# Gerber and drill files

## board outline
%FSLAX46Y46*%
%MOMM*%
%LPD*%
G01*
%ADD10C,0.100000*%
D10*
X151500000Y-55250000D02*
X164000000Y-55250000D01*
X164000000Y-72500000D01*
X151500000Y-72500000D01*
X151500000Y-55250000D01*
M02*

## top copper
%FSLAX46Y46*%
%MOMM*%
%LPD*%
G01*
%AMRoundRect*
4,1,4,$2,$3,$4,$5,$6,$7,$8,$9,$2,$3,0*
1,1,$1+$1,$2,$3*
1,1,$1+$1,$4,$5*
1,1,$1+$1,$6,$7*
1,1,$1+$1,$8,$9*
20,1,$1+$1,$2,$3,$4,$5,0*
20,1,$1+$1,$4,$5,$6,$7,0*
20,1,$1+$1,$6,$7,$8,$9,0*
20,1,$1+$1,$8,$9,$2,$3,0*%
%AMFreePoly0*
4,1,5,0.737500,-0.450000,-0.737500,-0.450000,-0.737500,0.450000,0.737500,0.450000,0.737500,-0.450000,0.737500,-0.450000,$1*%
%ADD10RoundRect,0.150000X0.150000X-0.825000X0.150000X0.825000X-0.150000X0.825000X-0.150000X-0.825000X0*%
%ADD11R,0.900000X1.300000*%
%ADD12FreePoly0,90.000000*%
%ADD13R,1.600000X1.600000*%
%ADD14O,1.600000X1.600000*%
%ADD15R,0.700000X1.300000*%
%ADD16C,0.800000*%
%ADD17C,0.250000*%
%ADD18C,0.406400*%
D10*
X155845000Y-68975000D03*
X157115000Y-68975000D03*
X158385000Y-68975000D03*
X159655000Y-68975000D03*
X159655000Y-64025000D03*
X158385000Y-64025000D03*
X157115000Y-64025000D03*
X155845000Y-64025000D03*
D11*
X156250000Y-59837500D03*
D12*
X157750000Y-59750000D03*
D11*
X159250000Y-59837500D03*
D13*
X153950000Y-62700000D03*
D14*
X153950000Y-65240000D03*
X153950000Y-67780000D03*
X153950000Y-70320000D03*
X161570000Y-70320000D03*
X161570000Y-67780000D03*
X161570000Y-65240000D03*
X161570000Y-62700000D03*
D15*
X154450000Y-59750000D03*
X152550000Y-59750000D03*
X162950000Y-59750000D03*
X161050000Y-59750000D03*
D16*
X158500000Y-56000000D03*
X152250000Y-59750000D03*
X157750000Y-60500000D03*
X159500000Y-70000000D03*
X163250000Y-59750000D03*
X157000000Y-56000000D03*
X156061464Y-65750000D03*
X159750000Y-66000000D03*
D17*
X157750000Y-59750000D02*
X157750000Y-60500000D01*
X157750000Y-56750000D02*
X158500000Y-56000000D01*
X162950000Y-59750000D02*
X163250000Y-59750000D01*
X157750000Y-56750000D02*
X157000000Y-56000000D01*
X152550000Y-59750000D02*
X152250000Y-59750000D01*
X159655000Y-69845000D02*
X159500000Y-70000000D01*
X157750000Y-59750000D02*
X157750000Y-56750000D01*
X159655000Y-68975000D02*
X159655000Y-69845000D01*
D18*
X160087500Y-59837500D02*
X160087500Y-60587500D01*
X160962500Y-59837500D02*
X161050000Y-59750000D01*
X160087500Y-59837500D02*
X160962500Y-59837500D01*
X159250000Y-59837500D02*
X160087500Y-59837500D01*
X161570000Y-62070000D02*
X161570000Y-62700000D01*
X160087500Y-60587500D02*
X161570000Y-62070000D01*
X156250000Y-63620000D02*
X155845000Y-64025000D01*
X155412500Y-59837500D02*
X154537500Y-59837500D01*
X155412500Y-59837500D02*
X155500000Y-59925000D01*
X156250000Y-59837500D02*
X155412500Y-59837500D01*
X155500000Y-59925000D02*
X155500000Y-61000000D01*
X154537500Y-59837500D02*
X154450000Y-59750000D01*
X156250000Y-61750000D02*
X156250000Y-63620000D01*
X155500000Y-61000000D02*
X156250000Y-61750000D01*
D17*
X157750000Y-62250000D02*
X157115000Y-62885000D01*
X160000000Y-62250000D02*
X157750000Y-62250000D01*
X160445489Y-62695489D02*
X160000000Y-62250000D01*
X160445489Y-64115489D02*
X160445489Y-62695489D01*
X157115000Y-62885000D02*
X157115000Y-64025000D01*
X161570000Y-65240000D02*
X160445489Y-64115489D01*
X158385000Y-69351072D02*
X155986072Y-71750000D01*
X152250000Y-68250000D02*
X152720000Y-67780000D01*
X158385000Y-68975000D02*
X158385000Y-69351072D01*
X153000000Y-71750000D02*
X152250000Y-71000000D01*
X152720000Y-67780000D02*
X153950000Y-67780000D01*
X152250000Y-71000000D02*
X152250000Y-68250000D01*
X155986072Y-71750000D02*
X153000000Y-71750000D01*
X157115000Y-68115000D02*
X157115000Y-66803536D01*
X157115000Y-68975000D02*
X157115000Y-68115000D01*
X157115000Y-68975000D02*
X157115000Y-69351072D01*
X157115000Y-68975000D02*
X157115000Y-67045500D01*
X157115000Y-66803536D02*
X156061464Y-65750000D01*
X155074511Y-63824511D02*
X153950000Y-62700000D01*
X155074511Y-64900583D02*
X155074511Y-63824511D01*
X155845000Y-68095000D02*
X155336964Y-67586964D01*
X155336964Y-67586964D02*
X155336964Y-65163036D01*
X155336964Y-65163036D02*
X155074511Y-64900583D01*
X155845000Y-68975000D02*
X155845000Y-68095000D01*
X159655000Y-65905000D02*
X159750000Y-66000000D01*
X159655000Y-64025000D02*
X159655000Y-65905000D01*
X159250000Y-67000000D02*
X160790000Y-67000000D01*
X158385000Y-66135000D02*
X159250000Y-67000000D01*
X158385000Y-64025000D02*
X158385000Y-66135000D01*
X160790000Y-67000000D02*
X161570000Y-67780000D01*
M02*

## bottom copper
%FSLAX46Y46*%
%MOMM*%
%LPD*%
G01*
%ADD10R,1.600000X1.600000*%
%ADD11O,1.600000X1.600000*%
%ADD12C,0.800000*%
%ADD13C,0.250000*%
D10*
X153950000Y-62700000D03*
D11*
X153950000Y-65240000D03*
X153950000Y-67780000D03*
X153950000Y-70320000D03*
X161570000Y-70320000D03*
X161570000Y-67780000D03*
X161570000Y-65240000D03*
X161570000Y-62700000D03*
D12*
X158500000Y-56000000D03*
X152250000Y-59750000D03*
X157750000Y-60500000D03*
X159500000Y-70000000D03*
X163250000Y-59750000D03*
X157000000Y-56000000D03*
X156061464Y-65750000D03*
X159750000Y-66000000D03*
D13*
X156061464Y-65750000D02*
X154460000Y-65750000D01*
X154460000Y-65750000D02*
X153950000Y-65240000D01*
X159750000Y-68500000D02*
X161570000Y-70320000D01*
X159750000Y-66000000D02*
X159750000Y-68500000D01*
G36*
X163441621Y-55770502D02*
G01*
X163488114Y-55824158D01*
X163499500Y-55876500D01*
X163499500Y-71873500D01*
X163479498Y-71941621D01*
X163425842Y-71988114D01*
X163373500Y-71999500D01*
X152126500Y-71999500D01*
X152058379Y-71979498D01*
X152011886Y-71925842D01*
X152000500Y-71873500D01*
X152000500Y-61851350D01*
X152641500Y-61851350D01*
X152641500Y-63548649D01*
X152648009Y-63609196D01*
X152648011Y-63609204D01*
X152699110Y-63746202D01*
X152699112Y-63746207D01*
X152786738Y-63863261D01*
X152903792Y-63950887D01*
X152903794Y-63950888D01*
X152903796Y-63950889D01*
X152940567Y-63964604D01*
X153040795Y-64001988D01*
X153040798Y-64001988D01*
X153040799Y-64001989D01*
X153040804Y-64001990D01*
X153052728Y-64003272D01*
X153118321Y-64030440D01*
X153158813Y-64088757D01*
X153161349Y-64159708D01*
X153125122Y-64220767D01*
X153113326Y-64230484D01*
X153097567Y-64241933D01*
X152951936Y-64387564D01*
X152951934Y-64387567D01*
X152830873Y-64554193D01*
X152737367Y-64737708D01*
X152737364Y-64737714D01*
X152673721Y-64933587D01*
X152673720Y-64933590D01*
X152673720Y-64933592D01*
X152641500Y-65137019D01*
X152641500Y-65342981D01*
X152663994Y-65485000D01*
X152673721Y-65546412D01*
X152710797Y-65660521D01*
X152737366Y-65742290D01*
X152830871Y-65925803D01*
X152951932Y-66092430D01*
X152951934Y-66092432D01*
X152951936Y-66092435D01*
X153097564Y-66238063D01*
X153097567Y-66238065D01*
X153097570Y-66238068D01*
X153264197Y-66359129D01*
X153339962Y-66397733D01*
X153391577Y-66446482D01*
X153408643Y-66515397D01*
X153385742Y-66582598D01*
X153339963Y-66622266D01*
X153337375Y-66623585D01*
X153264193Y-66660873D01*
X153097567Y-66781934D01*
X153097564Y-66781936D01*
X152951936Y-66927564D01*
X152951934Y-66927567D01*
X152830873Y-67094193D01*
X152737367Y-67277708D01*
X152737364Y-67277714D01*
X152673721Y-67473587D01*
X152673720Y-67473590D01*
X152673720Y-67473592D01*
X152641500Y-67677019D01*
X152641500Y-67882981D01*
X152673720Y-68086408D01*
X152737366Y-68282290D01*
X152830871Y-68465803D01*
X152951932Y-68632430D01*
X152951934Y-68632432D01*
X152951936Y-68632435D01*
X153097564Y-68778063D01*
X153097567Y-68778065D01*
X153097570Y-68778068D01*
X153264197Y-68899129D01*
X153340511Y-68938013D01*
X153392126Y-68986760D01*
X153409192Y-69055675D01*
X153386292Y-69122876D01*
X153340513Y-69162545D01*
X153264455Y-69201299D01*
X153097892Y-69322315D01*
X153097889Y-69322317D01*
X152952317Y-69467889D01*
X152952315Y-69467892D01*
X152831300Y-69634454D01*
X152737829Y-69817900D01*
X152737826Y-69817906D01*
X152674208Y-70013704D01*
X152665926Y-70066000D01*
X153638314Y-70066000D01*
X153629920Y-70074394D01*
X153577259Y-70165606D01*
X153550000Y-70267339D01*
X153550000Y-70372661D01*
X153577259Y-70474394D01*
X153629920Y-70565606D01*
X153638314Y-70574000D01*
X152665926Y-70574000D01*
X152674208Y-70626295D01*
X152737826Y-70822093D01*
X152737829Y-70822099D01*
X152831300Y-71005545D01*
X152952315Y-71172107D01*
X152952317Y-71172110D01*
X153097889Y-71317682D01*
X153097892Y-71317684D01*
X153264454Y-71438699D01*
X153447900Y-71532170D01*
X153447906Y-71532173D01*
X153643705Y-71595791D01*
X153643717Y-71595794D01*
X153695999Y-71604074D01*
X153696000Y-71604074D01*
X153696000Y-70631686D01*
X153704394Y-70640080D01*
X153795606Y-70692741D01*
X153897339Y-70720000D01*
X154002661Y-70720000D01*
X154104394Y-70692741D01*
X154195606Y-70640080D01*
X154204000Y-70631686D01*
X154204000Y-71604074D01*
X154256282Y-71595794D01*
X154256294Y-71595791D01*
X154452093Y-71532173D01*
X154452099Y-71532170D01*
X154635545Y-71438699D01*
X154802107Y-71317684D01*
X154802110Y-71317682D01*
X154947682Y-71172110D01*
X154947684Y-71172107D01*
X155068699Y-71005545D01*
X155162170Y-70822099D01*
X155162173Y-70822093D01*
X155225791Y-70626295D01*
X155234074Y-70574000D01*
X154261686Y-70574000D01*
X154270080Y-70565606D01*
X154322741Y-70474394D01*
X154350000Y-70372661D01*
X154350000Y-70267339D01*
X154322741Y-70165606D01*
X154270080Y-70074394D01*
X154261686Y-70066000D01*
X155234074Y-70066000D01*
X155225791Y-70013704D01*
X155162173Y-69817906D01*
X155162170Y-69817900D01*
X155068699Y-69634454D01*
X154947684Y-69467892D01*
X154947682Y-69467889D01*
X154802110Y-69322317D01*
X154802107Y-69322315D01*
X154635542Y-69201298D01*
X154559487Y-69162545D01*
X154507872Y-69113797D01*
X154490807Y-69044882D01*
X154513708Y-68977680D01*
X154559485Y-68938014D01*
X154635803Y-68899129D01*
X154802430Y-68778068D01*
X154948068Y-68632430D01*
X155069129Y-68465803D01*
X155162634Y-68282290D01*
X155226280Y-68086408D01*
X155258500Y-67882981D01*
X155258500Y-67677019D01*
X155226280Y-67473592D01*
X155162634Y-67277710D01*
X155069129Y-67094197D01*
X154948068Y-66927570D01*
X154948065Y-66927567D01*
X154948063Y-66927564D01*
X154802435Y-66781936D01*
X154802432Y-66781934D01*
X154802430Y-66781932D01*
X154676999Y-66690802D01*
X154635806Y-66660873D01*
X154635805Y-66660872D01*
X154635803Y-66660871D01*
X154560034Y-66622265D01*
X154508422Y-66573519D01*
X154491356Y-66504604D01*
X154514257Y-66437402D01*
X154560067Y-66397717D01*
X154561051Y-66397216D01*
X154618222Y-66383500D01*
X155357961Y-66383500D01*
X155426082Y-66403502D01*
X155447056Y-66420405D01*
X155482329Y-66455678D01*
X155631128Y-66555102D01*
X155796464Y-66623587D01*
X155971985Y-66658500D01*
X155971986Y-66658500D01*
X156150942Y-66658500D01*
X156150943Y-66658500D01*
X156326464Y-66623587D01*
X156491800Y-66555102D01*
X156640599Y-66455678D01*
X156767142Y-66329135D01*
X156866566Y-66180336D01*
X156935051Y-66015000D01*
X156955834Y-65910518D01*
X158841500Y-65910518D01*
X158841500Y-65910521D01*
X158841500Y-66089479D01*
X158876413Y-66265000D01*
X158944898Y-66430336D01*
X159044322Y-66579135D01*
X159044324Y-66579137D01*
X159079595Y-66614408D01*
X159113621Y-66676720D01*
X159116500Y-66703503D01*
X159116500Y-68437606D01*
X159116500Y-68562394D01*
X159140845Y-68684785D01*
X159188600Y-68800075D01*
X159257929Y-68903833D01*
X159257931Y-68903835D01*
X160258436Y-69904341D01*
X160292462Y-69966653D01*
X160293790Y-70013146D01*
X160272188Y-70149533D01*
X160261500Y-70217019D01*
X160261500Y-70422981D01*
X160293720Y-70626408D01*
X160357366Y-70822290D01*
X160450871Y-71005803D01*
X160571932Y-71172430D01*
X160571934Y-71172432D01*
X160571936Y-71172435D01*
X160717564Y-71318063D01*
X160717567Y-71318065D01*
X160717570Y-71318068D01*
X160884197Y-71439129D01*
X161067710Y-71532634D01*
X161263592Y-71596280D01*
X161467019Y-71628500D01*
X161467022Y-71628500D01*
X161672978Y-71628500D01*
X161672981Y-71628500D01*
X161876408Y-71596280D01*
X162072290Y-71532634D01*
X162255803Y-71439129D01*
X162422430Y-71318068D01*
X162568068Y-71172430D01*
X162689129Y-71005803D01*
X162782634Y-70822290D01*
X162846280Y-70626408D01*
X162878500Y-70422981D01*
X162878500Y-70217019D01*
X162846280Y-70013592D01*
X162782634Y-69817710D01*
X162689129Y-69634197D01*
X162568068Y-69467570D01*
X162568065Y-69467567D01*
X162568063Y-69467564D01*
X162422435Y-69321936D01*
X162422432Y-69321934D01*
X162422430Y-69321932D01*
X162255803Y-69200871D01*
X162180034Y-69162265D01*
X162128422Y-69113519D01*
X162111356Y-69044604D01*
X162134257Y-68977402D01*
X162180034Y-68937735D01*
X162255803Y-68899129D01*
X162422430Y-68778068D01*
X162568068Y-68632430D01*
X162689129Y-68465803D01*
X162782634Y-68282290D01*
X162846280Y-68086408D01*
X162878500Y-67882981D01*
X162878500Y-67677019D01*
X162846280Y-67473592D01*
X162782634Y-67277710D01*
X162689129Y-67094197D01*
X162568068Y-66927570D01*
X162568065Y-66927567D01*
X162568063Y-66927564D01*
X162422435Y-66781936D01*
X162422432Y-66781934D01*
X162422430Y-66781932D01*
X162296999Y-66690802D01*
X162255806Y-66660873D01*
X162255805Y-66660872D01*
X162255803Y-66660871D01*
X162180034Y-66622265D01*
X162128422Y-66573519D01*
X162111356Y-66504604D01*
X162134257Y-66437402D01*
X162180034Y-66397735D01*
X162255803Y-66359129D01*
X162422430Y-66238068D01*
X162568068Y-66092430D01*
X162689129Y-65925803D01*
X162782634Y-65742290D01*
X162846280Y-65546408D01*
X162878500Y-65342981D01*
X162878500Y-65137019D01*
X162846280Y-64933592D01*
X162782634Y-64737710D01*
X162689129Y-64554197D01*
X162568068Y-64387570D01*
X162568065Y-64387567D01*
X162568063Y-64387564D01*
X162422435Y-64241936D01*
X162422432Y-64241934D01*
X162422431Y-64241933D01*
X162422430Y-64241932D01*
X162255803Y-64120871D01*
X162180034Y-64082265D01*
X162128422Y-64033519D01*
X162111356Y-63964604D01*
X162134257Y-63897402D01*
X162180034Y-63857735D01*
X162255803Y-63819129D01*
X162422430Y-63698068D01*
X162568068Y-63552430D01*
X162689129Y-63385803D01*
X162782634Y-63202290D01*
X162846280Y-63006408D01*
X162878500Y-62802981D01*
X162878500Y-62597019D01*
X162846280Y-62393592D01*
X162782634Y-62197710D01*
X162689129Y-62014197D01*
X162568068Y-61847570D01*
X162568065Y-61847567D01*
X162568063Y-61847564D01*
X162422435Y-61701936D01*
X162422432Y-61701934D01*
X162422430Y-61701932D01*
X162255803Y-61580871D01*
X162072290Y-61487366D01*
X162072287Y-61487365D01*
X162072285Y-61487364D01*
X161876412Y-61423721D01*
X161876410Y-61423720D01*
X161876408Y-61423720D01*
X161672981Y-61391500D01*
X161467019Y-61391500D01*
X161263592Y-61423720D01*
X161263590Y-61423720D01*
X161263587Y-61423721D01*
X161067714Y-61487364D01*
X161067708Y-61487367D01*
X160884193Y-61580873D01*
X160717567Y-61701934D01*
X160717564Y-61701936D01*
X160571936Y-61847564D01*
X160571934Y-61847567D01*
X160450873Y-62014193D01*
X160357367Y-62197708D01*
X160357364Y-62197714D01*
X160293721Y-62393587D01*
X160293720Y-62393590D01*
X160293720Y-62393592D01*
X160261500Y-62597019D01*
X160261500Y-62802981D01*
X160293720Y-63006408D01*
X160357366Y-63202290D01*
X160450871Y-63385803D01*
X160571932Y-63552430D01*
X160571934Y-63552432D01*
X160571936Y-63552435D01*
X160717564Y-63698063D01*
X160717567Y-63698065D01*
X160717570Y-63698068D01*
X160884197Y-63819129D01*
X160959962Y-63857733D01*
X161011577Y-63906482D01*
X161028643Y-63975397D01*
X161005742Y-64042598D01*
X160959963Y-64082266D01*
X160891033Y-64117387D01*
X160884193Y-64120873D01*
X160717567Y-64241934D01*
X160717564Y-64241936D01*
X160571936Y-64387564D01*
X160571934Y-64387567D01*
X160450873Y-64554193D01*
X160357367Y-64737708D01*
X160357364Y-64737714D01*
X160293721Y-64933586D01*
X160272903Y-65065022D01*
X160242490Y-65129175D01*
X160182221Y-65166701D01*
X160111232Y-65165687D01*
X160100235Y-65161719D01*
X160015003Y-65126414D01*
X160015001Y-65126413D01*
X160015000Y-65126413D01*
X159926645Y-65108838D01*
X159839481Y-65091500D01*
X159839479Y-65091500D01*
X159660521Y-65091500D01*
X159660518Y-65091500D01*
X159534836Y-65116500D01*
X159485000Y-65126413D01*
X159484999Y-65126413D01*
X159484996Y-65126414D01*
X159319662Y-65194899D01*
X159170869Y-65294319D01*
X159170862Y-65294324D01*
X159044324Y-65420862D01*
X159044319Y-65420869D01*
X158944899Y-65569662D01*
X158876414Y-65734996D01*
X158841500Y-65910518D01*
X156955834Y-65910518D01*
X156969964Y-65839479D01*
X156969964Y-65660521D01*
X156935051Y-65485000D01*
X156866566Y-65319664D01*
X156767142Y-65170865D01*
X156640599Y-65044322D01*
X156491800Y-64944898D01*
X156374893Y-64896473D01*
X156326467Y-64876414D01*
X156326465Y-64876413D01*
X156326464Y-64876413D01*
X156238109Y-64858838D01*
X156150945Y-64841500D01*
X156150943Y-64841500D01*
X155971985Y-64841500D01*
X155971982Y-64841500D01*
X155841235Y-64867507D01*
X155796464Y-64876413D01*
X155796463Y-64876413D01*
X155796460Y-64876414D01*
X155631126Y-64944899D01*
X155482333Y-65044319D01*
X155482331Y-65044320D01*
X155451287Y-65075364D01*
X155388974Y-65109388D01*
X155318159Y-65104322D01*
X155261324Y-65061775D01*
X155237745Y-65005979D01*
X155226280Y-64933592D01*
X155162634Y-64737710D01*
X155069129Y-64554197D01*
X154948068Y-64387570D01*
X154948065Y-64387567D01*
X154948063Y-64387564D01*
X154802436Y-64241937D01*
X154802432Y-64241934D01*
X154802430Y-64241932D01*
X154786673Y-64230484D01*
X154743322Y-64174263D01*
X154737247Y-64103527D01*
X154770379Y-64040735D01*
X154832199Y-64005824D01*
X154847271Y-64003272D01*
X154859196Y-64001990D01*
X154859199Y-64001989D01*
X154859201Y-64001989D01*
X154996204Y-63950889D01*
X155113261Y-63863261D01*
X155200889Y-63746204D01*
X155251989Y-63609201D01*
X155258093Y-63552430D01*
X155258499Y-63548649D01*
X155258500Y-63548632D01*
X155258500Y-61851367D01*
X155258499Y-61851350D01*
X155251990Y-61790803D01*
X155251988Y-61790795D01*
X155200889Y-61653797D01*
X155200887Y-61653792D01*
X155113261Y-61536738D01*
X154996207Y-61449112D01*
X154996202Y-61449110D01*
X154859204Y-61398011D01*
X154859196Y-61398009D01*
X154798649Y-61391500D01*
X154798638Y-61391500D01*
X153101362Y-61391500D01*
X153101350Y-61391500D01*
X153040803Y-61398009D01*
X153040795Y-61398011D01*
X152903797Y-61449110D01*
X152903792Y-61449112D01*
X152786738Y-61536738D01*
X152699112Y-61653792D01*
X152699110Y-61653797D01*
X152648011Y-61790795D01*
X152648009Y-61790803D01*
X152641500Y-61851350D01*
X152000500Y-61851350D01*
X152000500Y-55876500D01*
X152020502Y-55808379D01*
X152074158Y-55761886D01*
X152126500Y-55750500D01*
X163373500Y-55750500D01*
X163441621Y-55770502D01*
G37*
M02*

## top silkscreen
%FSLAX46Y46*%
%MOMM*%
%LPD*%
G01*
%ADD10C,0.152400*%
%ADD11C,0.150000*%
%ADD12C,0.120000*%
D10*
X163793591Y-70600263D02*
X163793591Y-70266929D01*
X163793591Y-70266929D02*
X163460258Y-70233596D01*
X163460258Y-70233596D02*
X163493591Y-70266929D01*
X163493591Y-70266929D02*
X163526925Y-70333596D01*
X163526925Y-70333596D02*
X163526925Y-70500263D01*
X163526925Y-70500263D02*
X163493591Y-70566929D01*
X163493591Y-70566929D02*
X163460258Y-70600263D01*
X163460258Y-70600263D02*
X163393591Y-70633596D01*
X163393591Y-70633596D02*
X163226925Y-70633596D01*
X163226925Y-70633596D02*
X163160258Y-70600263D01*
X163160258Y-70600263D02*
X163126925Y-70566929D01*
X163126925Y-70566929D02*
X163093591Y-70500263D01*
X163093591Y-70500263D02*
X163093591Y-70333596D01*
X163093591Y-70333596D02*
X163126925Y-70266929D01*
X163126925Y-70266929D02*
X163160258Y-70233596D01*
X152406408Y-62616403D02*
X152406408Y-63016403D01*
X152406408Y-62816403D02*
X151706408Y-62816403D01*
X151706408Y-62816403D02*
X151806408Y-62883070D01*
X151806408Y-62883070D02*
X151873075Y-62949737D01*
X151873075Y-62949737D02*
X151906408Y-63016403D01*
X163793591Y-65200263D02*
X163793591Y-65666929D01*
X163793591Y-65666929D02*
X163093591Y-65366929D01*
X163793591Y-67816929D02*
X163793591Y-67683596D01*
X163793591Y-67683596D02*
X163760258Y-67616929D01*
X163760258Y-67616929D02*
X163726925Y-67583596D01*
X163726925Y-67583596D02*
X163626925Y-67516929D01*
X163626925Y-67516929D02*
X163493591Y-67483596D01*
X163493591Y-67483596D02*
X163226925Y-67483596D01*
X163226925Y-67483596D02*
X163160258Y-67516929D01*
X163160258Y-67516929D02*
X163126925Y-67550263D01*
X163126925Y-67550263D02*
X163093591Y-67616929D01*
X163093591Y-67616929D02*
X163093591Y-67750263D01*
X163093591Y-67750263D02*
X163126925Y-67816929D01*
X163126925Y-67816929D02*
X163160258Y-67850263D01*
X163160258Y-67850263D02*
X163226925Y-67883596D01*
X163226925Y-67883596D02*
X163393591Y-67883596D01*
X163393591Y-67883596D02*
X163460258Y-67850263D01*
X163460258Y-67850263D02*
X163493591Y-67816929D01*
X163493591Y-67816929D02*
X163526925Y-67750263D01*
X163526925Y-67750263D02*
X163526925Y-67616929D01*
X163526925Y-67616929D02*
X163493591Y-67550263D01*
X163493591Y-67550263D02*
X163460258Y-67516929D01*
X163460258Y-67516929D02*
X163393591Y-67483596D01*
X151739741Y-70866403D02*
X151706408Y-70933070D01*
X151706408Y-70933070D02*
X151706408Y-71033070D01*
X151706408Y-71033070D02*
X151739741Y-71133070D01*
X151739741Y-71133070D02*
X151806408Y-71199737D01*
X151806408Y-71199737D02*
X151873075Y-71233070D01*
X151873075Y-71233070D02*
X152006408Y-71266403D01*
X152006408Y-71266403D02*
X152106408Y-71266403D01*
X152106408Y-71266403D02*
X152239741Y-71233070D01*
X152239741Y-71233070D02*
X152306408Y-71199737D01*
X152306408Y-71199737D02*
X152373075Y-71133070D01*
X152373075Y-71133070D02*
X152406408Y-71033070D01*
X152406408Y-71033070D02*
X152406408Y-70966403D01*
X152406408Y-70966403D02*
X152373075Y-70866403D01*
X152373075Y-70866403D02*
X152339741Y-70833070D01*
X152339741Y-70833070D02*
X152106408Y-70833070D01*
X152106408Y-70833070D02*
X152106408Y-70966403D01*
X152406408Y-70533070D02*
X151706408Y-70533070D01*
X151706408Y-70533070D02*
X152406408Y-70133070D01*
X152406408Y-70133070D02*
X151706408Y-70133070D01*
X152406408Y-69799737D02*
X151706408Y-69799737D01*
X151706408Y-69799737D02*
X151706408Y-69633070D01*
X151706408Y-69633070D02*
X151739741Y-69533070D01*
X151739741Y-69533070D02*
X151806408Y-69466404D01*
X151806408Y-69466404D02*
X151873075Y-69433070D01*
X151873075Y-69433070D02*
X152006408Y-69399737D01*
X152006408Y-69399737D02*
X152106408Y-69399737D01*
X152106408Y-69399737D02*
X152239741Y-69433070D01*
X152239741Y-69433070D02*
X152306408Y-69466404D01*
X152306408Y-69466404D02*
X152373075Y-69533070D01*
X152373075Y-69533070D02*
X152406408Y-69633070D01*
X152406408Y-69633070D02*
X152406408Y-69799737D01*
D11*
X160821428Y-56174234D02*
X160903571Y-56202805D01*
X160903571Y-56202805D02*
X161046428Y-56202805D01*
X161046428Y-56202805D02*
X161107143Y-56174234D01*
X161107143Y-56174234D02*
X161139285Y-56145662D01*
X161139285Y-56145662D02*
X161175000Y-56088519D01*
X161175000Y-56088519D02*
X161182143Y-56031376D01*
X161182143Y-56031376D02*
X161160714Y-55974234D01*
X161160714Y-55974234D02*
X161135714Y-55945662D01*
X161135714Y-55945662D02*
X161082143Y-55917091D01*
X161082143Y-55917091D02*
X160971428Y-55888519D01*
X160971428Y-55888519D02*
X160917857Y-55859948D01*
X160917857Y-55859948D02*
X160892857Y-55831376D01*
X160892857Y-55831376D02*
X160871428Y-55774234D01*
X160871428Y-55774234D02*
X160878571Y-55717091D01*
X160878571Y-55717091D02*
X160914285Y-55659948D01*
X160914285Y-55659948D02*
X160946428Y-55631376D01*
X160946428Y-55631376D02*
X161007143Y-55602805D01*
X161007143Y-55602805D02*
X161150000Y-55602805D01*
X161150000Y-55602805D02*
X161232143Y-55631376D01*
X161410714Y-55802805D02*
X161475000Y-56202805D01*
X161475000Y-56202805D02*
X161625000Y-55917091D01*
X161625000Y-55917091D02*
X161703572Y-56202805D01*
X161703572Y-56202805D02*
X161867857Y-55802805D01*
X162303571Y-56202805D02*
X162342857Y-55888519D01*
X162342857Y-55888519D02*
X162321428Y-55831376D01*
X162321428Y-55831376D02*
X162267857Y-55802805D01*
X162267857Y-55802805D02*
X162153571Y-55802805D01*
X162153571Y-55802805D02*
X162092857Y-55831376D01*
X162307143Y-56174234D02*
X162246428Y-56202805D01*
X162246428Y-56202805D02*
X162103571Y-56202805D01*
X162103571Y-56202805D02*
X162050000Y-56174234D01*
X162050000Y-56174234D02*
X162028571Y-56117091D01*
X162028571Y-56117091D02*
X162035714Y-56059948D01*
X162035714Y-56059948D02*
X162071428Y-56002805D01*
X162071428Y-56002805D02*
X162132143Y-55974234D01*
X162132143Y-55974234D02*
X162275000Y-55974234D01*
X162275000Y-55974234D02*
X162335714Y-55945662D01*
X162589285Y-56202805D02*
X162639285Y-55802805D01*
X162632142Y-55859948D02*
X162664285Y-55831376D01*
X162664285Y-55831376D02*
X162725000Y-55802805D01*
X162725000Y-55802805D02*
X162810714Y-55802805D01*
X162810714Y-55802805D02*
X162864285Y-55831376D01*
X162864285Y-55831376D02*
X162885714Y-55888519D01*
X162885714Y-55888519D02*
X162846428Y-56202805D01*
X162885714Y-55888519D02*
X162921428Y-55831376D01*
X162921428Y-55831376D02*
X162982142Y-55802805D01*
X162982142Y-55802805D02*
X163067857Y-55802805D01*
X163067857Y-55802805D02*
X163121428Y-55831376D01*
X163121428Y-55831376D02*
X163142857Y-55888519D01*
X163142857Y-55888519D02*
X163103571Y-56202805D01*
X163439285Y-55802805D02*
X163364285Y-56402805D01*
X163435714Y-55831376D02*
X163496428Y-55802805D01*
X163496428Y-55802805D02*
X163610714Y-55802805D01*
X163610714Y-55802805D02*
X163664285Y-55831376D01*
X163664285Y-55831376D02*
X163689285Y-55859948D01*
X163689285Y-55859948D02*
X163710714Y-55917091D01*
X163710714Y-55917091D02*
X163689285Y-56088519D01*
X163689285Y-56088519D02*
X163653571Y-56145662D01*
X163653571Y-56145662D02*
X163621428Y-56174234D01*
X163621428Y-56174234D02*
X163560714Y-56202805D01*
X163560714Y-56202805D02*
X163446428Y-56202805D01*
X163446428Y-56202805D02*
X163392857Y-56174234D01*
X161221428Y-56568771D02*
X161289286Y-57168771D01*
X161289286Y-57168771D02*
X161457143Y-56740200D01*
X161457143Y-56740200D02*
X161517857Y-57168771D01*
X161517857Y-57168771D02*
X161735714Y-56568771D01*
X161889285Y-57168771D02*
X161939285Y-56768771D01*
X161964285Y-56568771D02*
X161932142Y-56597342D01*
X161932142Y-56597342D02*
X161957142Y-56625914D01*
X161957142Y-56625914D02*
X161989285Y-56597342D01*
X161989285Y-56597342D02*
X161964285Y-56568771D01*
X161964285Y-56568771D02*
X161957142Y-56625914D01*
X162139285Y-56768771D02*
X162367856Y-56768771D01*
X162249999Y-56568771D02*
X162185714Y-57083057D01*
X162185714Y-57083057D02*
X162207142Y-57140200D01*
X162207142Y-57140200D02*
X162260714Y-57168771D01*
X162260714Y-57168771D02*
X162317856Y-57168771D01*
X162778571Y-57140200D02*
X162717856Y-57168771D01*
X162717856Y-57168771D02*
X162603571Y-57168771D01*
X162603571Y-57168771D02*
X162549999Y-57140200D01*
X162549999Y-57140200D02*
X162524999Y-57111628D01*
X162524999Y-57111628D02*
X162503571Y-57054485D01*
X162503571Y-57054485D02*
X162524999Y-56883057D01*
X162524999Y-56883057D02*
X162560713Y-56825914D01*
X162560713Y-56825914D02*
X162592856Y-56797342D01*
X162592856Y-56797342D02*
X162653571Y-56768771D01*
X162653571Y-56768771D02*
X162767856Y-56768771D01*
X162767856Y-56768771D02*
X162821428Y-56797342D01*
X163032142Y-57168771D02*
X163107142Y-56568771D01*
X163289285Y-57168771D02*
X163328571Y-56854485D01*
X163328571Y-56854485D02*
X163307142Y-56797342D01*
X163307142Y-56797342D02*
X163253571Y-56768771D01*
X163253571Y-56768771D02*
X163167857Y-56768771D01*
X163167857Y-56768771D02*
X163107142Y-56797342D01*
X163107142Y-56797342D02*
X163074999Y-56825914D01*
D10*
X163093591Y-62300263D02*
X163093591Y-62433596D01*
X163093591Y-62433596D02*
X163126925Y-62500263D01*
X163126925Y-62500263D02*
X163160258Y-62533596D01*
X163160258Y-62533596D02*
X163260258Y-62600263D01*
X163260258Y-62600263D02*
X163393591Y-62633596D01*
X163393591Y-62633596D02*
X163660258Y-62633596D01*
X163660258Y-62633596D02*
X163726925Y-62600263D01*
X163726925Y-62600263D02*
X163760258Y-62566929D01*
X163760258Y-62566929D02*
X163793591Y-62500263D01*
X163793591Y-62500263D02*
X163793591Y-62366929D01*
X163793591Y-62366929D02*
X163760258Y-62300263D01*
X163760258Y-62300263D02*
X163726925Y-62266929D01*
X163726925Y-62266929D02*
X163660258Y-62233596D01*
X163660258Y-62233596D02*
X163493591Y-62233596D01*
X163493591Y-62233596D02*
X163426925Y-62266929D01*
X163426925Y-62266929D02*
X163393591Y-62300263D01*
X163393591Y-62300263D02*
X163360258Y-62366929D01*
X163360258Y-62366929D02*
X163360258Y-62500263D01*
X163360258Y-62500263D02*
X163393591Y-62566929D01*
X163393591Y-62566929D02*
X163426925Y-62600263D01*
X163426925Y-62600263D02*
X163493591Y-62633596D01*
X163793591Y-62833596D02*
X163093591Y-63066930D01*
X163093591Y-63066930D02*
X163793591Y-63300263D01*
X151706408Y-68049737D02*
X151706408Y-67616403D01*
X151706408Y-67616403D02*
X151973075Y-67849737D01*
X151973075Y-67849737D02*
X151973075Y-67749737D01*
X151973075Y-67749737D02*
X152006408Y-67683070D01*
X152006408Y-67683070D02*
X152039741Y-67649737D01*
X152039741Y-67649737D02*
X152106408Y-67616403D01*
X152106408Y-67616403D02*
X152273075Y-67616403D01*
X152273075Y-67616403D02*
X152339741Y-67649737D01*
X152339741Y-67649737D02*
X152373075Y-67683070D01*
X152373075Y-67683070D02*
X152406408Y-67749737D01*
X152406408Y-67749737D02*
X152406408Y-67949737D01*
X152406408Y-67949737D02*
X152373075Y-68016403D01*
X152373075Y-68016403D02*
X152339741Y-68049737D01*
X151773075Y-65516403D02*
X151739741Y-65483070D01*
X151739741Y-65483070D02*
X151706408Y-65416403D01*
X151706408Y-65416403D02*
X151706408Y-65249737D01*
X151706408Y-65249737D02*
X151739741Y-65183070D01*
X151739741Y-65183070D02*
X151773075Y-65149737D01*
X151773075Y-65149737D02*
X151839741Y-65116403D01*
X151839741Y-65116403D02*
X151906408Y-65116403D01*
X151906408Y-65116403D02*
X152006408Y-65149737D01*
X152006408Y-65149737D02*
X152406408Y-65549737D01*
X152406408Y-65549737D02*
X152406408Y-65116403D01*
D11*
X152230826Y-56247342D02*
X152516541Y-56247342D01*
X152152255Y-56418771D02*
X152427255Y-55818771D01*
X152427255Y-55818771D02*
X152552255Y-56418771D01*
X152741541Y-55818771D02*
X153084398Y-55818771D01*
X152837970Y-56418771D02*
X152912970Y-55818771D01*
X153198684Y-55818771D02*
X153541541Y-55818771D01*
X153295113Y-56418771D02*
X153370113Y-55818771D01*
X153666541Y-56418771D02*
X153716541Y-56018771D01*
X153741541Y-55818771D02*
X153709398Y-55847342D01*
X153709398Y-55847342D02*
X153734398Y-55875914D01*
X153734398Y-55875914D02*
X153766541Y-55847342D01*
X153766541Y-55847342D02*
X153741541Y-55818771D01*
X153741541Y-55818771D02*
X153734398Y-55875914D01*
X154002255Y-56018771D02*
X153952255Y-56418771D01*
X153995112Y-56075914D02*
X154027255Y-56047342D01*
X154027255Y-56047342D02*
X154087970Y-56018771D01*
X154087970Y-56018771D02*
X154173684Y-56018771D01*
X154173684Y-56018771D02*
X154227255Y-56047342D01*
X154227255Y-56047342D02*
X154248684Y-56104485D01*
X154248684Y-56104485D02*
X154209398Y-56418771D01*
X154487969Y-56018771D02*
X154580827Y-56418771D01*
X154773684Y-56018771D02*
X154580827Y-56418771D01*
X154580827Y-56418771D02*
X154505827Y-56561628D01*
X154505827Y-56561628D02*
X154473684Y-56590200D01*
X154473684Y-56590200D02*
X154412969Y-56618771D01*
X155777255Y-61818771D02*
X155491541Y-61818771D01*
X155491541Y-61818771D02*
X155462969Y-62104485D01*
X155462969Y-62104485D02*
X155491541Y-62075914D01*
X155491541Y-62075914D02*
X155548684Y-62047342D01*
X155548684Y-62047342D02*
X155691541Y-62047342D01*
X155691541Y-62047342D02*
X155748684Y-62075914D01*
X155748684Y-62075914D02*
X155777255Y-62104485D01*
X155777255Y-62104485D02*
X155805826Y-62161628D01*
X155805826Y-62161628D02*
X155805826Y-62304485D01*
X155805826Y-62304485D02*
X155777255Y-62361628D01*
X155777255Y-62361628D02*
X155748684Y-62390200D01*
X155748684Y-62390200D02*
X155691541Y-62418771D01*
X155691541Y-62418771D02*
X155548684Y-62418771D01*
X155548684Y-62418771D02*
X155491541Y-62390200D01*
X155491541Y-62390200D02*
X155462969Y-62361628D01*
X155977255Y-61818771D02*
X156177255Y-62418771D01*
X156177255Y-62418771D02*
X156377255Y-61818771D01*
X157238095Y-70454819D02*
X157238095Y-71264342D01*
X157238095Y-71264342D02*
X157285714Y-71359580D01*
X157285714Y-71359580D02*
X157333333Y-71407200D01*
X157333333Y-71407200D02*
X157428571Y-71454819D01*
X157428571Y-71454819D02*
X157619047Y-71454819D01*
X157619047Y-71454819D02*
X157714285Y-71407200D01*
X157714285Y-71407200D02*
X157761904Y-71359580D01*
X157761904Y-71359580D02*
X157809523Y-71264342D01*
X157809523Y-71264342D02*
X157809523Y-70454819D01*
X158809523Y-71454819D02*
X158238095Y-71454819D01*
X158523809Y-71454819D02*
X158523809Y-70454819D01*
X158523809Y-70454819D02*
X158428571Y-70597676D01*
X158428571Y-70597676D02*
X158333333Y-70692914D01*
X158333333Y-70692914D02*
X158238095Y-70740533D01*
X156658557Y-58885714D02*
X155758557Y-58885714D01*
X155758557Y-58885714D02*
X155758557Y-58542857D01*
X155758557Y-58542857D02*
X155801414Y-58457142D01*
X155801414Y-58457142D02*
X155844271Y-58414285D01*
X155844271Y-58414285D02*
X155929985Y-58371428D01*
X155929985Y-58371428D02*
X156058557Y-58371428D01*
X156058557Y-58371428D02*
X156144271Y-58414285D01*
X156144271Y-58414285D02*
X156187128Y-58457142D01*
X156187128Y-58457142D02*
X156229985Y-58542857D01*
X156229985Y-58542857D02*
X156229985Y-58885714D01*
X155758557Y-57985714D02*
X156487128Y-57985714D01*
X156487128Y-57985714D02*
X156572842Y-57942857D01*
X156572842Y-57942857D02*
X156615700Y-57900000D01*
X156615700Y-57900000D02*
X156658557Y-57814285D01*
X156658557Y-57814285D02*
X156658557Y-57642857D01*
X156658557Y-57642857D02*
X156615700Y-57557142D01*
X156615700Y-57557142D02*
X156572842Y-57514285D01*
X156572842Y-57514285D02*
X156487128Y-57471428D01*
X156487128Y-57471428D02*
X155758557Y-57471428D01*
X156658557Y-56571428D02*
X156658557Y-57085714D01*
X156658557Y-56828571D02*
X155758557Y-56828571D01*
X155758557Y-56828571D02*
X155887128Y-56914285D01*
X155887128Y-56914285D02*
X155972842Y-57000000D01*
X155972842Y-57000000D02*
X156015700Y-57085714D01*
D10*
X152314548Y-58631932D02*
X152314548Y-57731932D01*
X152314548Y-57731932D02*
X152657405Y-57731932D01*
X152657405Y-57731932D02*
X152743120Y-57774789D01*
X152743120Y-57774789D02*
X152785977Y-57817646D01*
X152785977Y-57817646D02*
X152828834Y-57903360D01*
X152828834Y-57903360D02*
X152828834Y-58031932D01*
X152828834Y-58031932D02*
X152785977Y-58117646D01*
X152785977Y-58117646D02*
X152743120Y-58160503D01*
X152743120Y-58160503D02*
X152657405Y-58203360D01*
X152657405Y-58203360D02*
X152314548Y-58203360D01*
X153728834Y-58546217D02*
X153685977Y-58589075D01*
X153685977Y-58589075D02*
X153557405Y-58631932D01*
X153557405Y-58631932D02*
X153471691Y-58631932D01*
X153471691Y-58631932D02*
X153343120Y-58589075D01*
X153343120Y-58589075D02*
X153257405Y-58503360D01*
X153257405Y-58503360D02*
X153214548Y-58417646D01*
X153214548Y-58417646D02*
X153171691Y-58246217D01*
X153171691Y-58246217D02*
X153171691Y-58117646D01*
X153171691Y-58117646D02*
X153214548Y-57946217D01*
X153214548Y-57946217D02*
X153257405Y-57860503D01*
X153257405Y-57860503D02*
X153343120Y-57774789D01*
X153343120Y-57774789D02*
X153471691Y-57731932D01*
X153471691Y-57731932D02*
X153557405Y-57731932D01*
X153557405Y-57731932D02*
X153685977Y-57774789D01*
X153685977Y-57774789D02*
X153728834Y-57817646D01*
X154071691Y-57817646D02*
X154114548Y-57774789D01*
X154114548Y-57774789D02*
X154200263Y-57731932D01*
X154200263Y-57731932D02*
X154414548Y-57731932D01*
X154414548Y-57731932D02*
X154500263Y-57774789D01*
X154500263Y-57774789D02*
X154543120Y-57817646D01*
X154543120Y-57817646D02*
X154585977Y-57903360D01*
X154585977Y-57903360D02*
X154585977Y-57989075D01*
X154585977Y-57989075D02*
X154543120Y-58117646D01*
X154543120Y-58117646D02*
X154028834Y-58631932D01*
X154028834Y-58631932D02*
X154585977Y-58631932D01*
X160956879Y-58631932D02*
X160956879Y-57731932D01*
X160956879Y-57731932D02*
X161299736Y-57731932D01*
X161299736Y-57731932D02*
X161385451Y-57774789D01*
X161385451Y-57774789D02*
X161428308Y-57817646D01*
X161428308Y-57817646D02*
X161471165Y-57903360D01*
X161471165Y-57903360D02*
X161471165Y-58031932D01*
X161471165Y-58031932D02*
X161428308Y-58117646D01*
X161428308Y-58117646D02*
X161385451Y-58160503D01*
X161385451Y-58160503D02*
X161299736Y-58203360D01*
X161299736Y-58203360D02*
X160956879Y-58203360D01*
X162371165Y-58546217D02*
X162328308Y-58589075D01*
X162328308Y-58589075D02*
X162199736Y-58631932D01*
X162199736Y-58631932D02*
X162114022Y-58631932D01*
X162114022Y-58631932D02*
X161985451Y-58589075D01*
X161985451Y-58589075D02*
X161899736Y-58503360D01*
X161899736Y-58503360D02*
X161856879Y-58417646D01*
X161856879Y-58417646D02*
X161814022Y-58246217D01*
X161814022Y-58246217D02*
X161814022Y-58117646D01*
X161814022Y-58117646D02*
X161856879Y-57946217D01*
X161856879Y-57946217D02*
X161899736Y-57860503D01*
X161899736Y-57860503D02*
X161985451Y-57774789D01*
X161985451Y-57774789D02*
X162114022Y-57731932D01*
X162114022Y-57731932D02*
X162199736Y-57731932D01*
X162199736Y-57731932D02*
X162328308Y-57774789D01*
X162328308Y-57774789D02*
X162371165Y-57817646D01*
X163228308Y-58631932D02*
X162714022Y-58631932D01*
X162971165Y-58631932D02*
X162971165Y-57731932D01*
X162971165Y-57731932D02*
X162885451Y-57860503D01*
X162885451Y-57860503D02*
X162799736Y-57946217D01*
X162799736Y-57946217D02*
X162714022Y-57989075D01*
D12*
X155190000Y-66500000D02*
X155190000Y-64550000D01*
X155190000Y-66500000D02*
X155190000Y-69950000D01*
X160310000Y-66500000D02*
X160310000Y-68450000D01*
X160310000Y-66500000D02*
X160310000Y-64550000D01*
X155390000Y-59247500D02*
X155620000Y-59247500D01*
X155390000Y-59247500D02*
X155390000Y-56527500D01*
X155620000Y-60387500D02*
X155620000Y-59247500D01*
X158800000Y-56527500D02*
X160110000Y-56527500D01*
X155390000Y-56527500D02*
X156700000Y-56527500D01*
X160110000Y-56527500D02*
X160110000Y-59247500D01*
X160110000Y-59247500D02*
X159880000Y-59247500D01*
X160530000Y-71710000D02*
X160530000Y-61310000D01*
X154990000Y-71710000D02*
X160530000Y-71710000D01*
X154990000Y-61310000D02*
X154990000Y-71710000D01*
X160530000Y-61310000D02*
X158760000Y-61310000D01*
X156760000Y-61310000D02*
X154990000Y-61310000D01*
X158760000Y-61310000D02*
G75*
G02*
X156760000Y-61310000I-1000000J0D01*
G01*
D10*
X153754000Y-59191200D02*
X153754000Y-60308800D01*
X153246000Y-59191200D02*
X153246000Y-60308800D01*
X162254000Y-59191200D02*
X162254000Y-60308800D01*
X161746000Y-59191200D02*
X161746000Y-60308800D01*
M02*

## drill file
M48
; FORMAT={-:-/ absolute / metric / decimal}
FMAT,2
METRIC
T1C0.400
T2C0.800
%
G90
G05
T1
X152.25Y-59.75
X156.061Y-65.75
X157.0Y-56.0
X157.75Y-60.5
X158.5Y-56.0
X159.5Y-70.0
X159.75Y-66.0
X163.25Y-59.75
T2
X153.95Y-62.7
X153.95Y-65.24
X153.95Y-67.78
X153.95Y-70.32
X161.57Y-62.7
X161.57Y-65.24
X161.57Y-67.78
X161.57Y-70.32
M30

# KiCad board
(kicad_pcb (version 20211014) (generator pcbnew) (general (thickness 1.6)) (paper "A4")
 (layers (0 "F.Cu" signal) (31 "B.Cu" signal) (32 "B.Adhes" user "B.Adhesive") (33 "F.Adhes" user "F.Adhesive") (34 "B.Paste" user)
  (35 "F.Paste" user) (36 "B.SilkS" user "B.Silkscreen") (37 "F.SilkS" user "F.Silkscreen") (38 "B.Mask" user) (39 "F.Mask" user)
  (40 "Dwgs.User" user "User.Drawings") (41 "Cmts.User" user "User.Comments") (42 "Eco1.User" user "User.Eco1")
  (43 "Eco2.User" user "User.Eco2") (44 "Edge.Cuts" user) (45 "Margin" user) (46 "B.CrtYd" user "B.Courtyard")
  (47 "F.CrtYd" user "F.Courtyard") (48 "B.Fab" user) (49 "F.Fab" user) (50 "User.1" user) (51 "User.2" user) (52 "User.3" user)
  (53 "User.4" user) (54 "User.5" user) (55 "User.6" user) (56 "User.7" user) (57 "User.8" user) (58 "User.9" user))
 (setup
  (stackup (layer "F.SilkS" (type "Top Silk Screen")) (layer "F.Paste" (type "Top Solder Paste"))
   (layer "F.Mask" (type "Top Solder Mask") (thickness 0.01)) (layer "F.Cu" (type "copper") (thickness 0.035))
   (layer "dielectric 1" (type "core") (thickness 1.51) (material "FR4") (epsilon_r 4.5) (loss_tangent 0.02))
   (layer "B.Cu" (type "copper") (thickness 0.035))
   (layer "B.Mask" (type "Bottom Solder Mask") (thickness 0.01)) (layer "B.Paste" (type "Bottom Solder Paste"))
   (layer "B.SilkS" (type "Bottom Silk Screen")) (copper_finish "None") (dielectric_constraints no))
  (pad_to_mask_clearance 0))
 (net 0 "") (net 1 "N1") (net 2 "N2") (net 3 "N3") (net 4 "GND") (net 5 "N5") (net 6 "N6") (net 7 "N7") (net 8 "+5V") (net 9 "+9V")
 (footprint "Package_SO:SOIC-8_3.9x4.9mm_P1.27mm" (layer "F.Cu") (at 157.75 66.5 90)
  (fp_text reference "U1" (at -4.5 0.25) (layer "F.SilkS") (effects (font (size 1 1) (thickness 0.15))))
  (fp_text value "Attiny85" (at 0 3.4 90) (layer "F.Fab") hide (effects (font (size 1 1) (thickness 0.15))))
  (fp_line (start 0 -2.56) (end 1.95 -2.56) (layer "F.SilkS") (width 0.12))
  (fp_line (start 0 -2.56) (end -3.45 -2.56) (layer "F.SilkS") (width 0.12))
  (fp_line (start 0 2.56) (end -1.95 2.56) (layer "F.SilkS") (width 0.12))
  (fp_line (start 0 2.56) (end 1.95 2.56) (layer "F.SilkS") (width 0.12))
  (pad "1" smd roundrect locked (at -2.475 -1.905 90) (size 1.95 0.6) (layers "F.Cu" "F.Paste" "F.Mask") (roundrect_rratio 0.25)
   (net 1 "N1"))
  (pad "2" smd roundrect locked (at -2.475 -0.635 90) (size 1.95 0.6) (layers "F.Cu" "F.Paste" "F.Mask") (roundrect_rratio 0.25)
   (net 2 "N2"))
  (pad "3" smd roundrect locked (at -2.475 0.635 90) (size 1.95 0.6) (layers "F.Cu" "F.Paste" "F.Mask") (roundrect_rratio 0.25) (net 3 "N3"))
  (pad "4" smd roundrect locked (at -2.475 1.905 90) (size 1.95 0.6) (layers "F.Cu" "F.Paste" "F.Mask") (roundrect_rratio 0.25)
   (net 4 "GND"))
  (pad "5" smd roundrect locked (at 2.475 1.905 90) (size 1.95 0.6) (layers "F.Cu" "F.Paste" "F.Mask") (roundrect_rratio 0.25) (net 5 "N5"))
  (pad "6" smd roundrect locked (at 2.475 0.635 90) (size 1.95 0.6) (layers "F.Cu" "F.Paste" "F.Mask") (roundrect_rratio 0.25) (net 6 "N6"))
  (pad "7" smd roundrect locked (at 2.475 -0.635 90) (size 1.95 0.6) (layers "F.Cu" "F.Paste" "F.Mask") (roundrect_rratio 0.25) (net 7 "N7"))
  (pad "8" smd roundrect locked (at 2.475 -1.905 90) (size 1.95 0.6) (layers "F.Cu" "F.Paste" "F.Mask") (roundrect_rratio 0.25)
   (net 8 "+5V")))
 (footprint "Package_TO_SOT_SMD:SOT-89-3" (layer "F.Cu") (at 157.75 58.1875 90)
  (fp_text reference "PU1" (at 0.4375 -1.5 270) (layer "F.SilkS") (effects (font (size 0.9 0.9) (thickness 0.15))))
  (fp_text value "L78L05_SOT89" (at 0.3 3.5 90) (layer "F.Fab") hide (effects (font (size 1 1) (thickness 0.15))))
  (fp_line (start -1.06 -2.36) (end -1.06 -2.13) (layer "F.SilkS") (width 0.12))
  (fp_line (start -1.06 -2.36) (end 1.66 -2.36) (layer "F.SilkS") (width 0.12))
  (fp_line (start -2.2 -2.13) (end -1.06 -2.13) (layer "F.SilkS") (width 0.12))
  (fp_line (start 1.66 1.05) (end 1.66 2.36) (layer "F.SilkS") (width 0.12))
  (fp_line (start 1.66 -2.36) (end 1.66 -1.05) (layer "F.SilkS") (width 0.12))
  (fp_line (start 1.66 2.36) (end -1.06 2.36) (layer "F.SilkS") (width 0.12))
  (fp_line (start -1.06 2.36) (end -1.06 2.13) (layer "F.SilkS") (width 0.12))
  (pad "1" smd rect locked (at -1.65 -1.5 90) (size 1.3 0.9) (layers "F.Cu" "F.Paste" "F.Mask") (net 8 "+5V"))
  (pad "2" smd custom locked (at -1.5625 0 90) (size 1.475 0.9) (layers "F.Cu" "F.Paste" "F.Mask") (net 4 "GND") (zone_connect 2)
   (options (clearance outline) (anchor rect)) (primitives))
  (pad "3" smd rect locked (at -1.65 1.5 90) (size 1.3 0.9) (layers "F.Cu" "F.Paste" "F.Mask") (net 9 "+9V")))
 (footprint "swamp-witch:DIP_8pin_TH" (layer "F.Cu") (at 153.95 62.7)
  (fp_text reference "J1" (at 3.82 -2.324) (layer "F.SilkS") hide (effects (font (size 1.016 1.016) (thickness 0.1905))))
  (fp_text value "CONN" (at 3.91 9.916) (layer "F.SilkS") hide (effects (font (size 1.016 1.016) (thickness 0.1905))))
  (fp_line (start 6.58 9.01) (end 6.58 -1.39) (layer "F.SilkS") (width 0.12))
  (fp_line (start 1.04 9.01) (end 6.58 9.01) (layer "F.SilkS") (width 0.12))
  (fp_line (start 1.04 -1.39) (end 1.04 9.01) (layer "F.SilkS") (width 0.12))
  (fp_line (start 6.58 -1.39) (end 4.81 -1.39) (layer "F.SilkS") (width 0.12))
  (fp_line (start 2.81 -1.39) (end 1.04 -1.39) (layer "F.SilkS") (width 0.12))
  (fp_arc (start 4.81 -1.39) (mid 3.81 -0.39) (end 2.81 -1.39) (layer "F.SilkS") (width 0.12))
  (pad "1" thru_hole rect locked (at 0 0) (size 1.6 1.6) (drill 0.8) (layers *.Cu *.Mask) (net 1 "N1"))
  (pad "2" thru_hole oval locked (at 0 2.54) (size 1.6 1.6) (drill 0.8) (layers *.Cu *.Mask) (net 2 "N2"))
  (pad "3" thru_hole oval locked (at 0 5.08) (size 1.6 1.6) (drill 0.8) (layers *.Cu *.Mask) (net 3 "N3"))
  (pad "4" thru_hole oval locked (at 0 7.62) (size 1.6 1.6) (drill 0.8) (layers *.Cu *.Mask) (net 4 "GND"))
  (pad "5" thru_hole oval locked (at 7.62 7.62) (size 1.6 1.6) (drill 0.8) (layers *.Cu *.Mask) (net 5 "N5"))
  (pad "6" thru_hole oval locked (at 7.62 5.08) (size 1.6 1.6) (drill 0.8) (layers *.Cu *.Mask) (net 6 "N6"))
  (pad "7" thru_hole oval locked (at 7.62 2.54) (size 1.6 1.6) (drill 0.8) (layers *.Cu *.Mask) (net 7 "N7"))
  (pad "8" thru_hole oval locked (at 7.62 0) (size 1.6 1.6) (drill 0.8) (layers *.Cu *.Mask) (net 9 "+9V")))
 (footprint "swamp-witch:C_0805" (layer "F.Cu") (at 153.5 59.75 180)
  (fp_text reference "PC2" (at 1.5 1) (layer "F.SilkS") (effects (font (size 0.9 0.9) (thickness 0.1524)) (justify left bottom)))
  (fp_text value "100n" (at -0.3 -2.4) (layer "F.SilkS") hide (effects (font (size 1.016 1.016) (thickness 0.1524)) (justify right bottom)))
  (fp_line (start -0.254 0.5588) (end -0.254 -0.5588) (layer "F.SilkS") (width 0.1524))
  (fp_line (start 0.254 0.5588) (end 0.254 -0.5588) (layer "F.SilkS") (width 0.1524))
  (pad "1" smd rect locked (at -0.95 0 180) (size 0.7 1.3) (layers "F.Cu" "F.Paste" "F.Mask") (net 8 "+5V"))
  (pad "2" smd rect locked (at 0.95 0 180) (size 0.7 1.3) (layers "F.Cu" "F.Paste" "F.Mask") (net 4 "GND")))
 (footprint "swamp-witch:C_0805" (layer "F.Cu") (at 162 59.75 180)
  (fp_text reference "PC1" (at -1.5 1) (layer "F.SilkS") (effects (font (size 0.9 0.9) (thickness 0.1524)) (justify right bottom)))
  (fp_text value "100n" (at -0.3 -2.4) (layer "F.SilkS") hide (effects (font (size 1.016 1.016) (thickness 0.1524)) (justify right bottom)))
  (fp_line (start -0.254 0.5588) (end -0.254 -0.5588) (layer "F.SilkS") (width 0.1524))
  (fp_line (start 0.254 0.5588) (end 0.254 -0.5588) (layer "F.SilkS") (width 0.1524))
  (pad "1" smd rect locked (at -0.95 0 180) (size 0.7 1.3) (layers "F.Cu" "F.Paste" "F.Mask") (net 4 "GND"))
  (pad "2" smd rect locked (at 0.95 0 180) (size 0.7 1.3) (layers "F.Cu" "F.Paste" "F.Mask") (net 9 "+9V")))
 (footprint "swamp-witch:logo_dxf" (layer "B.Cu") (at 166.355152 71.834907 180)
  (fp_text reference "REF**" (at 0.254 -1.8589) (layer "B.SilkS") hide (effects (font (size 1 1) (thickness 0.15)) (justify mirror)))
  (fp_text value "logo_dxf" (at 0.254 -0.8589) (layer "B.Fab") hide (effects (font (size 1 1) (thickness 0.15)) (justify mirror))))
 (gr_rect (start 151.5 55.25) (end 164 72.5) (layer "Edge.Cuts") (width 0.1) (fill none))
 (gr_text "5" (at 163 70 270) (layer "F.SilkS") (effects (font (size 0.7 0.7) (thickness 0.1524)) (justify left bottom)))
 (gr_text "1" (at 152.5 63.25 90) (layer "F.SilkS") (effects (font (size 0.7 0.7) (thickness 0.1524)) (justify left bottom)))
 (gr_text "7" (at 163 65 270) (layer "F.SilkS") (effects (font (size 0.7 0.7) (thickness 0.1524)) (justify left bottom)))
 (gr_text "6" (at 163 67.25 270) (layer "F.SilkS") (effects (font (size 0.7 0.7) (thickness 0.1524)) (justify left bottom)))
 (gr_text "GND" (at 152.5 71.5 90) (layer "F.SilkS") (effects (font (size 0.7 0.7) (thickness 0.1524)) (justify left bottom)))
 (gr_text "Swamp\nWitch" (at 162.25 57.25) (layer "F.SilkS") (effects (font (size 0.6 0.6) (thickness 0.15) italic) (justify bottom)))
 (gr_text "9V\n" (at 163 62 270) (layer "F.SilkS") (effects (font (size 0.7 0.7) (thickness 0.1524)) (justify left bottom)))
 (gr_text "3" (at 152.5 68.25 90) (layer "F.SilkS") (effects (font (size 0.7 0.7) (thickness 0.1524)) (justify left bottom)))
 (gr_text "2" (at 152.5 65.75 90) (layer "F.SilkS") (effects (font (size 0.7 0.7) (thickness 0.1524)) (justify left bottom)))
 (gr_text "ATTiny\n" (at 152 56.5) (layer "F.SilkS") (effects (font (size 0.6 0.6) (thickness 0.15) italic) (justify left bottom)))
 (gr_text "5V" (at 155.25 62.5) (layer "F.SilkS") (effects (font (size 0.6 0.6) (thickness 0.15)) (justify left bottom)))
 (segment (start 157.75 59.75) (end 157.75 60.5) (width 0.25) (layer "F.Cu") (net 4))
 (segment (start 157.75 56.75) (end 158.5 56) (width 0.25) (layer "F.Cu") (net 4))
 (segment (start 162.95 59.75) (end 163.25 59.75) (width 0.25) (layer "F.Cu") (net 4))
 (segment (start 157.75 56.75) (end 157 56) (width 0.25) (layer "F.Cu") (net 4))
 (segment (start 152.55 59.75) (end 152.25 59.75) (width 0.25) (layer "F.Cu") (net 4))
 (segment (start 159.655 69.845) (end 159.5 70) (width 0.25) (layer "F.Cu") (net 4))
 (segment (start 157.75 59.75) (end 157.75 56.75) (width 0.25) (layer "F.Cu") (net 4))
 (segment (start 159.655 68.975) (end 159.655 69.845) (width 0.25) (layer "F.Cu") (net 4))
 (via (at 158.5 56) (size 0.8) (drill 0.4) (layers "F.Cu" "B.Cu") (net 4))
 (via (at 152.25 59.75) (size 0.8) (drill 0.4) (layers "F.Cu" "B.Cu") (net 4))
 (via (at 157.75 60.5) (size 0.8) (drill 0.4) (layers "F.Cu" "B.Cu") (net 4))
 (via (at 159.5 70) (size 0.8) (drill 0.4) (layers "F.Cu" "B.Cu") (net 4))
 (via (at 163.25 59.75) (size 0.8) (drill 0.4) (layers "F.Cu" "B.Cu") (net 4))
 (via (at 157 56) (size 0.8) (drill 0.4) (layers "F.Cu" "B.Cu") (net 4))
 (segment (start 160.0875 59.8375) (end 160.0875 60.5875) (width 0.4064) (layer "F.Cu") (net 9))
 (segment (start 160.9625 59.8375) (end 161.05 59.75) (width 0.4064) (layer "F.Cu") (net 9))
 (segment (start 160.0875 59.8375) (end 160.9625 59.8375) (width 0.4064) (layer "F.Cu") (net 9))
 (segment (start 159.25 59.8375) (end 160.0875 59.8375) (width 0.4064) (layer "F.Cu") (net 9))
 (segment (start 161.57 62.07) (end 161.57 62.7) (width 0.4064) (layer "F.Cu") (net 9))
 (segment (start 160.0875 60.5875) (end 161.57 62.07) (width 0.4064) (layer "F.Cu") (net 9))
 (segment (start 156.25 63.62) (end 155.845 64.025) (width 0.4064) (layer "F.Cu") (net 8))
 (segment (start 155.4125 59.8375) (end 154.5375 59.8375) (width 0.4064) (layer "F.Cu") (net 8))
 (segment (start 155.4125 59.8375) (end 155.5 59.925) (width 0.4064) (layer "F.Cu") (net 8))
 (segment (start 156.25 59.8375) (end 155.4125 59.8375) (width 0.4064) (layer "F.Cu") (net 8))
 (segment (start 155.5 59.925) (end 155.5 61) (width 0.4064) (layer "F.Cu") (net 8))
 (segment (start 154.5375 59.8375) (end 154.45 59.75) (width 0.4064) (layer "F.Cu") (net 8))
 (segment (start 156.25 61.75) (end 156.25 63.62) (width 0.4064) (layer "F.Cu") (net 8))
 (segment (start 155.5 61) (end 156.25 61.75) (width 0.4064) (layer "F.Cu") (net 8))
 (segment (start 157.75 62.25) (end 157.115 62.885) (width 0.25) (layer "F.Cu") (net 7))
 (segment (start 160 62.25) (end 157.75 62.25) (width 0.25) (layer "F.Cu") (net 7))
 (segment (start 160.445489 62.695489) (end 160 62.25) (width 0.25) (layer "F.Cu") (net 7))
 (segment (start 160.445489 64.115489) (end 160.445489 62.695489) (width 0.25) (layer "F.Cu") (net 7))
 (segment (start 157.115 62.885) (end 157.115 64.025) (width 0.25) (layer "F.Cu") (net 7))
 (segment (start 161.57 65.24) (end 160.445489 64.115489) (width 0.25) (layer "F.Cu") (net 7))
 (segment (start 158.385 69.351072) (end 155.986072 71.75) (width 0.25) (layer "F.Cu") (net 3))
 (segment (start 152.25 68.25) (end 152.72 67.78) (width 0.25) (layer "F.Cu") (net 3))
 (segment (start 158.385 68.975) (end 158.385 69.351072) (width 0.25) (layer "F.Cu") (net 3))
 (segment (start 153 71.75) (end 152.25 71) (width 0.25) (layer "F.Cu") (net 3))
 (segment (start 152.72 67.78) (end 153.95 67.78) (width 0.25) (layer "F.Cu") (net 3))
 (segment (start 152.25 71) (end 152.25 68.25) (width 0.25) (layer "F.Cu") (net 3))
 (segment (start 155.986072 71.75) (end 153 71.75) (width 0.25) (layer "F.Cu") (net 3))
 (segment (start 157.115 68.115) (end 157.115 66.803536) (width 0.25) (layer "F.Cu") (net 2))
 (segment (start 157.115 68.975) (end 157.115 68.115) (width 0.25) (layer "F.Cu") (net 2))
 (segment (start 157.115 68.975) (end 157.115 69.351072) (width 0.25) (layer "F.Cu") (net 2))
 (segment (start 157.115 68.975) (end 157.115 67.0455) (width 0.25) (layer "F.Cu") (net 2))
 (segment (start 157.115 66.803536) (end 156.061464 65.75) (width 0.25) (layer "F.Cu") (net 2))
 (via (at 156.061464 65.75) (size 0.8) (drill 0.4) (layers "F.Cu" "B.Cu") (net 2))
 (segment (start 156.061464 65.75) (end 154.46 65.75) (width 0.25) (layer "B.Cu") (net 2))
 (segment (start 154.46 65.75) (end 153.95 65.24) (width 0.25) (layer "B.Cu") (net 2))
 (segment (start 155.074511 63.824511) (end 153.95 62.7) (width 0.25) (layer "F.Cu") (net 1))
 (segment (start 155.074511 64.900583) (end 155.074511 63.824511) (width 0.25) (layer "F.Cu") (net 1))
 (segment (start 155.845 68.095) (end 155.336964 67.586964) (width 0.25) (layer "F.Cu") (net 1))
 (segment (start 155.336964 67.586964) (end 155.336964 65.163036) (width 0.25) (layer "F.Cu") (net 1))
 (segment (start 155.336964 65.163036) (end 155.074511 64.900583) (width 0.25) (layer "F.Cu") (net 1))
 (segment (start 155.845 68.975) (end 155.845 68.095) (width 0.25) (layer "F.Cu") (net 1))
 (segment (start 159.655 65.905) (end 159.75 66) (width 0.25) (layer "F.Cu") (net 5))
 (segment (start 159.655 64.025) (end 159.655 65.905) (width 0.25) (layer "F.Cu") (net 5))
 (via (at 159.75 66) (size 0.8) (drill 0.4) (layers "F.Cu" "B.Cu") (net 5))
 (segment (start 159.75 68.5) (end 161.57 70.32) (width 0.25) (layer "B.Cu") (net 5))
 (segment (start 159.75 66) (end 159.75 68.5) (width 0.25) (layer "B.Cu") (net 5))
 (segment (start 159.25 67) (end 160.79 67) (width 0.25) (layer "F.Cu") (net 6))
 (segment (start 158.385 66.135) (end 159.25 67) (width 0.25) (layer "F.Cu") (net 6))
 (segment (start 158.385 64.025) (end 158.385 66.135) (width 0.25) (layer "F.Cu") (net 6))
 (segment (start 160.79 67) (end 161.57 67.78) (width 0.25) (layer "F.Cu") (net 6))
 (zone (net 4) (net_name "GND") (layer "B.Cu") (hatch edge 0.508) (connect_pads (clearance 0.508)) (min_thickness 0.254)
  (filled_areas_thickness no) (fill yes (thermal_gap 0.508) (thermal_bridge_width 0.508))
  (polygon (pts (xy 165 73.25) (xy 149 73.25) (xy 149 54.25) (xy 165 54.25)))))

